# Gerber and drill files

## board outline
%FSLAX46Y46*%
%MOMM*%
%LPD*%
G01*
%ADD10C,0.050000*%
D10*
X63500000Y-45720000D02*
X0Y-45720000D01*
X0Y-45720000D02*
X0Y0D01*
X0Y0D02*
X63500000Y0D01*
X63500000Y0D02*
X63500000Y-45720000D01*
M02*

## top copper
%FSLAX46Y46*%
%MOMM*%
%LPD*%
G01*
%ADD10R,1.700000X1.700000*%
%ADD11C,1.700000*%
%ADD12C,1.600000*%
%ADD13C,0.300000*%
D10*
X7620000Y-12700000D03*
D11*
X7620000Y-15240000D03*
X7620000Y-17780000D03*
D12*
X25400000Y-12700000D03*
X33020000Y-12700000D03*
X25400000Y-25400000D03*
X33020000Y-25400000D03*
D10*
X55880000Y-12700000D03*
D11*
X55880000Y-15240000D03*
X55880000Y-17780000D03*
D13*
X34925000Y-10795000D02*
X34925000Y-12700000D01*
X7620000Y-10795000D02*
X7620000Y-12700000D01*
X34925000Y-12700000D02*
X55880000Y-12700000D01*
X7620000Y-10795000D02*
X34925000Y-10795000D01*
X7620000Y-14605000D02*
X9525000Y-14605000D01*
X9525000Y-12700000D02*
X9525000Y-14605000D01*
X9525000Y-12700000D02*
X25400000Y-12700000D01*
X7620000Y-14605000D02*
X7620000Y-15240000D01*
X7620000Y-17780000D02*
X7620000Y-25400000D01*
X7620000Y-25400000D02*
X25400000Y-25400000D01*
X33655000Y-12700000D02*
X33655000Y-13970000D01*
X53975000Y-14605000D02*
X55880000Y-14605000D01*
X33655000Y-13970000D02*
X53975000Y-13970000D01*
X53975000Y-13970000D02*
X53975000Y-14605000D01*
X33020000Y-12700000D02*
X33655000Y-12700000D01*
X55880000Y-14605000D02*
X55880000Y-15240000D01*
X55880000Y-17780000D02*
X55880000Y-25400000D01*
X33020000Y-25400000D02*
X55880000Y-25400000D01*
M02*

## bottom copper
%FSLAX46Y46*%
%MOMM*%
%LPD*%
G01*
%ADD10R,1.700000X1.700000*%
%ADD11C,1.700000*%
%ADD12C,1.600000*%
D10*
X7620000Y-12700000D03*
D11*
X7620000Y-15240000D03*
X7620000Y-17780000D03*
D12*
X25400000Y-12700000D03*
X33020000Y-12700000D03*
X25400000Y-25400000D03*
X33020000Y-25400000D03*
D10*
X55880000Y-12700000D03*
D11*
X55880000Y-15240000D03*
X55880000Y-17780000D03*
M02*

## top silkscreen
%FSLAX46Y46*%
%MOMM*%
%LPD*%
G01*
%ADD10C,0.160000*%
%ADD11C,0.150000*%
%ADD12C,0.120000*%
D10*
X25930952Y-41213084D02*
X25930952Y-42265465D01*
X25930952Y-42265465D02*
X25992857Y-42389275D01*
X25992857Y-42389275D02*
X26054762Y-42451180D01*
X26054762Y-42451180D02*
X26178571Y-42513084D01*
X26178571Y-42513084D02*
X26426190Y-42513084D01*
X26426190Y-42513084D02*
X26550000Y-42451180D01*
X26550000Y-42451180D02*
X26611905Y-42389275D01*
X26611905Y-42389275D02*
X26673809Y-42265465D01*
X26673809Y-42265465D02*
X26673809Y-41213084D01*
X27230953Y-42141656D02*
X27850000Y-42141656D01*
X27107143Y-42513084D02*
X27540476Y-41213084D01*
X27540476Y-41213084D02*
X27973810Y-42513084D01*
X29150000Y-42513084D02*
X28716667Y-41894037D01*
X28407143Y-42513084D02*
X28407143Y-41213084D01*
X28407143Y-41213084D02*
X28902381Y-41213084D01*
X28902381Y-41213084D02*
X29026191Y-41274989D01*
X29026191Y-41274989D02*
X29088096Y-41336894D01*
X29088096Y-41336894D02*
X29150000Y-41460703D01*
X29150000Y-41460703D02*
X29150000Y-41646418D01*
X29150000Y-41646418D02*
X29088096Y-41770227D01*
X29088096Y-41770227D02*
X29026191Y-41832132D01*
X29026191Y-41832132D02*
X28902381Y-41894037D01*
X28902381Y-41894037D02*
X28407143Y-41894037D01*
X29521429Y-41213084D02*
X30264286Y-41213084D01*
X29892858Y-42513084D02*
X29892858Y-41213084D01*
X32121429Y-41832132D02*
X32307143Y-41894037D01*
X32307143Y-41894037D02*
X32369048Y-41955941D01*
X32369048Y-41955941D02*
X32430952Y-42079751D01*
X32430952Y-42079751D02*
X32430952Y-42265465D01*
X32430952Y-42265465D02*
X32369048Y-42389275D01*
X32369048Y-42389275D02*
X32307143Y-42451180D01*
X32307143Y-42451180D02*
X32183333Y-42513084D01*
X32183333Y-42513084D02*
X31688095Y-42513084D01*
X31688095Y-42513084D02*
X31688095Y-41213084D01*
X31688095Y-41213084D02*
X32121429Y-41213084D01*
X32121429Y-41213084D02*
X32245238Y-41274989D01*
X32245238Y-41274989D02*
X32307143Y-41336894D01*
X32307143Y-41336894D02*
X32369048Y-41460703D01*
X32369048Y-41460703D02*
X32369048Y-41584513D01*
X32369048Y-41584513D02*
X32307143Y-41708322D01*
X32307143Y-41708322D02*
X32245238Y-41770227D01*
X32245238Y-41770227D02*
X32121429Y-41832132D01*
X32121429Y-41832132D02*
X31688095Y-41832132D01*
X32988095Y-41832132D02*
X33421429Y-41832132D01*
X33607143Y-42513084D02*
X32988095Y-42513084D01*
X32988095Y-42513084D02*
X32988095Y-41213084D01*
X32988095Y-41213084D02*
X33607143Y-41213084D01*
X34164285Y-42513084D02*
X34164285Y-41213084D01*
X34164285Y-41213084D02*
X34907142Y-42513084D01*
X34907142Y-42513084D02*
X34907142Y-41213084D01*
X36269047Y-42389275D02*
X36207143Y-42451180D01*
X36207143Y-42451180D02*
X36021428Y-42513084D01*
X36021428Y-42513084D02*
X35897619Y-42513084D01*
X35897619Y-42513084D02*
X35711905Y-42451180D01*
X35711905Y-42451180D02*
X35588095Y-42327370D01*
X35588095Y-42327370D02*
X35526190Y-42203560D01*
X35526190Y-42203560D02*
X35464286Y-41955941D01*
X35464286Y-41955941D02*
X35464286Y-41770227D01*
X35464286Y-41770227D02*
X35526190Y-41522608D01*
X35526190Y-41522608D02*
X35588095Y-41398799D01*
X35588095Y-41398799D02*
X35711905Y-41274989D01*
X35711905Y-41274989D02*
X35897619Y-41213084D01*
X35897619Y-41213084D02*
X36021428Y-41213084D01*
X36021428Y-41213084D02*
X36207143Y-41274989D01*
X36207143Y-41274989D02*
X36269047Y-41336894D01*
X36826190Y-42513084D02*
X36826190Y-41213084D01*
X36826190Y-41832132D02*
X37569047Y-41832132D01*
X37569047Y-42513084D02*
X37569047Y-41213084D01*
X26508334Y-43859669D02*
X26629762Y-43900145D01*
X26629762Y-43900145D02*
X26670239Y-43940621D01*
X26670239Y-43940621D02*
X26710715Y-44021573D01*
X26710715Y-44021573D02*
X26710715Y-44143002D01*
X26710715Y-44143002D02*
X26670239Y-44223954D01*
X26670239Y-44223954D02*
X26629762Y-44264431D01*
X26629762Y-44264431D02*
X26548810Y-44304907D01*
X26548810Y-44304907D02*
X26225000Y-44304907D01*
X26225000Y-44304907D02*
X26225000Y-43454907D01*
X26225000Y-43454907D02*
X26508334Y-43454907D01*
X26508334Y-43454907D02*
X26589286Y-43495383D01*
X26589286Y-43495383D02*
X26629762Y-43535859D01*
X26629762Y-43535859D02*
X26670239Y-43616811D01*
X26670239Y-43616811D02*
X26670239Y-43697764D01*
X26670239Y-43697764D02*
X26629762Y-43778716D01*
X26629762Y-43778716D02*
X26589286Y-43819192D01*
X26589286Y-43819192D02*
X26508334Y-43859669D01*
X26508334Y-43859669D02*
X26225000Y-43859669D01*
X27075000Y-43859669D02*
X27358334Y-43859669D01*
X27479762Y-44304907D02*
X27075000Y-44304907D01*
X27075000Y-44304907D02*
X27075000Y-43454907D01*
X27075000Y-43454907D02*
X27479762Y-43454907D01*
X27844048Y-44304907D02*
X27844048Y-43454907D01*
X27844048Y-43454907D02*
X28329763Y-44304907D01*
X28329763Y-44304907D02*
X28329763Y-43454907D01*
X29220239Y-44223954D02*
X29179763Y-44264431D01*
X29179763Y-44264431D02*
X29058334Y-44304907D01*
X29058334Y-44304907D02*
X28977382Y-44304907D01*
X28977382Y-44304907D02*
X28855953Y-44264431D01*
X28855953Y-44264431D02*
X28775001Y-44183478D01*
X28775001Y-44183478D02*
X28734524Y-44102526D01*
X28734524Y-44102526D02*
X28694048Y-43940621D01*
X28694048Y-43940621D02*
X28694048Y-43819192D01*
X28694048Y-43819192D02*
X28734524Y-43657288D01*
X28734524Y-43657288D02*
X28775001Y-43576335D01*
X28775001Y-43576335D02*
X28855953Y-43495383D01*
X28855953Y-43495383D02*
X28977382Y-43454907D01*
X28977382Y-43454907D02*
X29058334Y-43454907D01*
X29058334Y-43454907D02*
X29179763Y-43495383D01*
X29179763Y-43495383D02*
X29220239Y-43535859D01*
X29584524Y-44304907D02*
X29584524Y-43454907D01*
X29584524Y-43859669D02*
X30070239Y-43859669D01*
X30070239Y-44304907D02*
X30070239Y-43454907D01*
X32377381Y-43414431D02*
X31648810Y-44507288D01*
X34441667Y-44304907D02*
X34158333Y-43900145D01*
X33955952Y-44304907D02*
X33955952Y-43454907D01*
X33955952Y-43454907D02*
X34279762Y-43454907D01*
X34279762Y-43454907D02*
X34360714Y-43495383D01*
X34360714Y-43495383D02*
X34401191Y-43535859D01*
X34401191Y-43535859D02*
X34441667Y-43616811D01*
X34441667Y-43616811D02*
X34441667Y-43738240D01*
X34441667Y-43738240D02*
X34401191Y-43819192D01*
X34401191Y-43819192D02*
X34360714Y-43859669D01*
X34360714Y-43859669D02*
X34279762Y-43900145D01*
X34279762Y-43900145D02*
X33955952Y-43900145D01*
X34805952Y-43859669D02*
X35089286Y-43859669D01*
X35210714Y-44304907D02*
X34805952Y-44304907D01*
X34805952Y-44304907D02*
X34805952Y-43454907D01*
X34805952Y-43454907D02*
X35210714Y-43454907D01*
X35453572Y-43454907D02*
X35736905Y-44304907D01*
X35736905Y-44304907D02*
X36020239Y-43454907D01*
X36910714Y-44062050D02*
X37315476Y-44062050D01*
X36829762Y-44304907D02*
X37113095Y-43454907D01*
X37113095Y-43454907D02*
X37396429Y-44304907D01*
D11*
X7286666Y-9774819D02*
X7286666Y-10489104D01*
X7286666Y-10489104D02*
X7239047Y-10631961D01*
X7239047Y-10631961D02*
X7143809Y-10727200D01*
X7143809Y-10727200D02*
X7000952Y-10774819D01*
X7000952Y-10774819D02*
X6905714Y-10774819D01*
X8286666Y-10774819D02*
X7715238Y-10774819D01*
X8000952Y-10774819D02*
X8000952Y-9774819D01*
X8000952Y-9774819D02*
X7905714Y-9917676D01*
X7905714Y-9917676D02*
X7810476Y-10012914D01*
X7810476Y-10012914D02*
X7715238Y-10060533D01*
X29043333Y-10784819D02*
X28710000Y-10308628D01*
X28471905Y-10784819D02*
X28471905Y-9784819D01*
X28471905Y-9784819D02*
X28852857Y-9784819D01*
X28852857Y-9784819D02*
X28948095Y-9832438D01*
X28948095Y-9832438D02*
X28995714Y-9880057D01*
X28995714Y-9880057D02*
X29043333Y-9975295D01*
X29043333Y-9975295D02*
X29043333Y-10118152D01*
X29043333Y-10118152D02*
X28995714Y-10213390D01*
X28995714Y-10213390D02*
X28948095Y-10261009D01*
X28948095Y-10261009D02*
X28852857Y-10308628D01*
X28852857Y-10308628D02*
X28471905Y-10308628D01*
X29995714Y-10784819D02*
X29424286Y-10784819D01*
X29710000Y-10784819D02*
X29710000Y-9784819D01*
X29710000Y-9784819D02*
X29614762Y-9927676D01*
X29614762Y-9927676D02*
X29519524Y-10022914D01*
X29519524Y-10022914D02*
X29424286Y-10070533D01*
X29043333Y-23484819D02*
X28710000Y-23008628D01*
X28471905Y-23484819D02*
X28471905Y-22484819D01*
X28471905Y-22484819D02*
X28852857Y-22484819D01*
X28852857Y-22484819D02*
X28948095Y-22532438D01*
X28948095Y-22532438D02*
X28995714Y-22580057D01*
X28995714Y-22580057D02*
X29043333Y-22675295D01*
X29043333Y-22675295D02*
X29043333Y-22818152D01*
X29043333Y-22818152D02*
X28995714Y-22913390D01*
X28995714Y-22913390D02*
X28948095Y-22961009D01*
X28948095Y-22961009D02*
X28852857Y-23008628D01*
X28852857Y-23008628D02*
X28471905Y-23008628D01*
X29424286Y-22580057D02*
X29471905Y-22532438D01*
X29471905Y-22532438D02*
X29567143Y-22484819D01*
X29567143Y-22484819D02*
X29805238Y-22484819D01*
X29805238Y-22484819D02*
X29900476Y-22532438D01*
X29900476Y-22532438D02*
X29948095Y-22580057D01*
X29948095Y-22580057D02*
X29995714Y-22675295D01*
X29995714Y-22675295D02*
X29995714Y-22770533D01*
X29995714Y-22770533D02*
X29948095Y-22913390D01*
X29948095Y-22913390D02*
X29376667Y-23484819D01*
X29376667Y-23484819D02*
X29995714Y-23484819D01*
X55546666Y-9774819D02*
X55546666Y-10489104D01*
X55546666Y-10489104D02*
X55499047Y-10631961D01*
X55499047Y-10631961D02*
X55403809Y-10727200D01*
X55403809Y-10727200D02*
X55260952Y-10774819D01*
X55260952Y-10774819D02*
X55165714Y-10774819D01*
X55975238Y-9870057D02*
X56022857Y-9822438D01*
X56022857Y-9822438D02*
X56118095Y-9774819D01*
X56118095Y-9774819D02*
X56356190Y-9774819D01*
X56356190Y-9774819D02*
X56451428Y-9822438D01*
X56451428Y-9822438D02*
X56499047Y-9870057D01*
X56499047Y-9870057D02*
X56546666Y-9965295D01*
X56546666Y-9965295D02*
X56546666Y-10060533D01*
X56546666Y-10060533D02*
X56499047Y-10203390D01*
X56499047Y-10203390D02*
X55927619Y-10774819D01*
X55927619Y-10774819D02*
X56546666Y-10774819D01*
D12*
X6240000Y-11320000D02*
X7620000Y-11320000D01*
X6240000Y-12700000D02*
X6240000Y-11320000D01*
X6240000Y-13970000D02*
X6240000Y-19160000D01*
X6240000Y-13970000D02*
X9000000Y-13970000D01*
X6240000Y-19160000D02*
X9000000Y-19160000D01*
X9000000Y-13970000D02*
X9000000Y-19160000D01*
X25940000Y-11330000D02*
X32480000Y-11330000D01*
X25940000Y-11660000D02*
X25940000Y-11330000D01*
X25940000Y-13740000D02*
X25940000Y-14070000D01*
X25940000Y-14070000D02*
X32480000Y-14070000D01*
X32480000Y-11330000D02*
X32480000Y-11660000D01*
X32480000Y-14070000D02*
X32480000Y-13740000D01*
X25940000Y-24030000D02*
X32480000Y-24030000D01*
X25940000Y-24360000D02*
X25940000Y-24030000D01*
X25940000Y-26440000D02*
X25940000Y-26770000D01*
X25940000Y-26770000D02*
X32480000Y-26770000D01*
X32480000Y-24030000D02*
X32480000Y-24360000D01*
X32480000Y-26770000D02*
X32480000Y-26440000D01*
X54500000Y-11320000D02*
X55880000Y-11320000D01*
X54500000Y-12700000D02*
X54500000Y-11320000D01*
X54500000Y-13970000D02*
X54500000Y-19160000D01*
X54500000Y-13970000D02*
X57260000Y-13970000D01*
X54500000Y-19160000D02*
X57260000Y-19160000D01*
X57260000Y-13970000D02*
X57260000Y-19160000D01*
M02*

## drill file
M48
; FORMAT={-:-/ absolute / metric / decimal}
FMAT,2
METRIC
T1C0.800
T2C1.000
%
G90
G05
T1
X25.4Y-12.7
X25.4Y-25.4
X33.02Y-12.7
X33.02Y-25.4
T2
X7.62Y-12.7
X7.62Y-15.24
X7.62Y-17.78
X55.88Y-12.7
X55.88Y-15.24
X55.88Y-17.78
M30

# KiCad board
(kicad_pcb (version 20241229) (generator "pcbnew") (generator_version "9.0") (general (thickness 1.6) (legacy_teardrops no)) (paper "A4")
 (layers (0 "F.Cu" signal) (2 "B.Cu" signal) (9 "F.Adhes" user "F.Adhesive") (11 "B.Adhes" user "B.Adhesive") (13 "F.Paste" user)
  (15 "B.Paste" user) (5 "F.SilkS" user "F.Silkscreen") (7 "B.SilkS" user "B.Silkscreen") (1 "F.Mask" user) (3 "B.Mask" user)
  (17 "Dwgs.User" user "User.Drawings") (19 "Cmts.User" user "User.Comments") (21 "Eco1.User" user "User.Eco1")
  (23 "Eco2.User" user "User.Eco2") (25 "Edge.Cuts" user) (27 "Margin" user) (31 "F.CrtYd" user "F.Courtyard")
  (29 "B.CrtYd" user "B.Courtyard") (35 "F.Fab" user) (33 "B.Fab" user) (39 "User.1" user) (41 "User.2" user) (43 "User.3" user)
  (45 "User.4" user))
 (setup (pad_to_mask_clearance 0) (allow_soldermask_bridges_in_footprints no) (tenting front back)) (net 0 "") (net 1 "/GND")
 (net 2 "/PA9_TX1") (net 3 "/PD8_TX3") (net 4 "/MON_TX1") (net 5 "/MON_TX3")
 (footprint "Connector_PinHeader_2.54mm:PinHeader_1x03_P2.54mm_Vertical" (layer "F.Cu") (at 7.62 12.7)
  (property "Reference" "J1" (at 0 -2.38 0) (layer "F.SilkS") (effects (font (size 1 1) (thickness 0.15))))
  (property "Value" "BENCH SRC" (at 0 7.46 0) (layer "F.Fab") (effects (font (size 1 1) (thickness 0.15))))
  (fp_line (start -1.38 -1.38) (end 0 -1.38) (stroke (width 0.12) (type solid)) (layer "F.SilkS"))
  (fp_line (start -1.38 0) (end -1.38 -1.38) (stroke (width 0.12) (type solid)) (layer "F.SilkS"))
  (fp_line (start -1.38 1.27) (end -1.38 6.46) (stroke (width 0.12) (type solid)) (layer "F.SilkS"))
  (fp_line (start -1.38 1.27) (end 1.38 1.27) (stroke (width 0.12) (type solid)) (layer "F.SilkS"))
  (fp_line (start -1.38 6.46) (end 1.38 6.46) (stroke (width 0.12) (type solid)) (layer "F.SilkS"))
  (fp_line (start 1.38 1.27) (end 1.38 6.46) (stroke (width 0.12) (type solid)) (layer "F.SilkS"))
  (pad "1" thru_hole rect (at 0 0) (size 1.7 1.7) (drill 1) (layers "*.Cu" "*.Mask") (remove_unused_layers no) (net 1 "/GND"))
  (pad "2" thru_hole circle (at 0 2.54) (size 1.7 1.7) (drill 1) (layers "*.Cu" "*.Mask") (remove_unused_layers no) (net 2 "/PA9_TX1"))
  (pad "3" thru_hole circle (at 0 5.08) (size 1.7 1.7) (drill 1) (layers "*.Cu" "*.Mask") (remove_unused_layers no) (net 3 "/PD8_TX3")))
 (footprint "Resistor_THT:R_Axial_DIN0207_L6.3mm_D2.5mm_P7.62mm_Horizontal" (layer "F.Cu") (at 25.4 12.7)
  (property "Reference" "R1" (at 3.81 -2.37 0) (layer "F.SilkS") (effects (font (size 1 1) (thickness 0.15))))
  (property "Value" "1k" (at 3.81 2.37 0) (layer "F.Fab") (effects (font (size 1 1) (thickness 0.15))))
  (fp_line (start 0.54 -1.37) (end 7.08 -1.37) (stroke (width 0.12) (type solid)) (layer "F.SilkS"))
  (fp_line (start 0.54 -1.04) (end 0.54 -1.37) (stroke (width 0.12) (type solid)) (layer "F.SilkS"))
  (fp_line (start 0.54 1.04) (end 0.54 1.37) (stroke (width 0.12) (type solid)) (layer "F.SilkS"))
  (fp_line (start 0.54 1.37) (end 7.08 1.37) (stroke (width 0.12) (type solid)) (layer "F.SilkS"))
  (fp_line (start 7.08 -1.37) (end 7.08 -1.04) (stroke (width 0.12) (type solid)) (layer "F.SilkS"))
  (fp_line (start 7.08 1.37) (end 7.08 1.04) (stroke (width 0.12) (type solid)) (layer "F.SilkS"))
  (pad "1" thru_hole circle (at 0 0) (size 1.6 1.6) (drill 0.8) (layers "*.Cu" "*.Mask") (remove_unused_layers no) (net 2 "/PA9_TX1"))
  (pad "2" thru_hole circle (at 7.62 0) (size 1.6 1.6) (drill 0.8) (layers "*.Cu" "*.Mask") (remove_unused_layers no) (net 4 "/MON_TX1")))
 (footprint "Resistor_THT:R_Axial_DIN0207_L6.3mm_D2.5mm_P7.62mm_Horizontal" (layer "F.Cu") (at 25.4 25.4)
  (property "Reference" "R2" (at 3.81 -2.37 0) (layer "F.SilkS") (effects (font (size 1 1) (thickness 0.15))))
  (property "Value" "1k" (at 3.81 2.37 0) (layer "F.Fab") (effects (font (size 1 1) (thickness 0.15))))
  (fp_line (start 0.54 -1.37) (end 7.08 -1.37) (stroke (width 0.12) (type solid)) (layer "F.SilkS"))
  (fp_line (start 0.54 -1.04) (end 0.54 -1.37) (stroke (width 0.12) (type solid)) (layer "F.SilkS"))
  (fp_line (start 0.54 1.04) (end 0.54 1.37) (stroke (width 0.12) (type solid)) (layer "F.SilkS"))
  (fp_line (start 0.54 1.37) (end 7.08 1.37) (stroke (width 0.12) (type solid)) (layer "F.SilkS"))
  (fp_line (start 7.08 -1.37) (end 7.08 -1.04) (stroke (width 0.12) (type solid)) (layer "F.SilkS"))
  (fp_line (start 7.08 1.37) (end 7.08 1.04) (stroke (width 0.12) (type solid)) (layer "F.SilkS"))
  (pad "1" thru_hole circle (at 0 0) (size 1.6 1.6) (drill 0.8) (layers "*.Cu" "*.Mask") (remove_unused_layers no) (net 3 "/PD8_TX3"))
  (pad "2" thru_hole circle (at 7.62 0) (size 1.6 1.6) (drill 0.8) (layers "*.Cu" "*.Mask") (remove_unused_layers no) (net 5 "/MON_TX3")))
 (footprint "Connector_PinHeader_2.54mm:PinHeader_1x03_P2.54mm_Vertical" (layer "F.Cu") (at 55.88 12.7)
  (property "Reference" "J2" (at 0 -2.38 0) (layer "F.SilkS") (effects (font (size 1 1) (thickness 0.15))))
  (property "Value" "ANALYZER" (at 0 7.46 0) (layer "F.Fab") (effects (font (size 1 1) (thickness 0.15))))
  (fp_line (start -1.38 -1.38) (end 0 -1.38) (stroke (width 0.12) (type solid)) (layer "F.SilkS"))
  (fp_line (start -1.38 0) (end -1.38 -1.38) (stroke (width 0.12) (type solid)) (layer "F.SilkS"))
  (fp_line (start -1.38 1.27) (end -1.38 6.46) (stroke (width 0.12) (type solid)) (layer "F.SilkS"))
  (fp_line (start -1.38 1.27) (end 1.38 1.27) (stroke (width 0.12) (type solid)) (layer "F.SilkS"))
  (fp_line (start -1.38 6.46) (end 1.38 6.46) (stroke (width 0.12) (type solid)) (layer "F.SilkS"))
  (fp_line (start 1.38 1.27) (end 1.38 6.46) (stroke (width 0.12) (type solid)) (layer "F.SilkS"))
  (pad "1" thru_hole rect (at 0 0) (size 1.7 1.7) (drill 1) (layers "*.Cu" "*.Mask") (remove_unused_layers no) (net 1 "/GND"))
  (pad "2" thru_hole circle (at 0 2.54) (size 1.7 1.7) (drill 1) (layers "*.Cu" "*.Mask") (remove_unused_layers no) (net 4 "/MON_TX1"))
  (pad "3" thru_hole circle (at 0 5.08) (size 1.7 1.7) (drill 1) (layers "*.Cu" "*.Mask") (remove_unused_layers no) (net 5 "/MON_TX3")))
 (gr_line (start 63.5 45.72) (end 0 45.72) (stroke (width 0.05) (type default)) (layer "Edge.Cuts"))
 (gr_line (start 0 45.72) (end 0 0) (stroke (width 0.05) (type default)) (layer "Edge.Cuts"))
 (gr_line (start 0 0) (end 63.5 0) (stroke (width 0.05) (type default)) (layer "Edge.Cuts"))
 (gr_line (start 63.5 0) (end 63.5 45.72) (stroke (width 0.05) (type default)) (layer "Edge.Cuts"))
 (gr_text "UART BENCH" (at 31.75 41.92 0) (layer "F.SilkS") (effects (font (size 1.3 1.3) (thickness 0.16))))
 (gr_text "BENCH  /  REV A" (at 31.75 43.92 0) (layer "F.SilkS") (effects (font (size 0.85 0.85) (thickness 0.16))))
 (segment (start 34.925 10.795) (end 34.925 12.7) (width 0.3) (layer "F.Cu") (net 1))
 (segment (start 7.62 10.795) (end 7.62 12.7) (width 0.3) (layer "F.Cu") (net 1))
 (segment (start 34.925 12.7) (end 55.88 12.7) (width 0.3) (layer "F.Cu") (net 1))
 (segment (start 7.62 10.795) (end 34.925 10.795) (width 0.3) (layer "F.Cu") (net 1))
 (segment (start 7.62 14.605) (end 9.525 14.605) (width 0.3) (layer "F.Cu") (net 2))
 (segment (start 9.525 12.7) (end 9.525 14.605) (width 0.3) (layer "F.Cu") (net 2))
 (segment (start 9.525 12.7) (end 25.4 12.7) (width 0.3) (layer "F.Cu") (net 2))
 (segment (start 7.62 14.605) (end 7.62 15.24) (width 0.3) (layer "F.Cu") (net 2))
 (segment (start 7.62 17.78) (end 7.62 25.4) (width 0.3) (layer "F.Cu") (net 3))
 (segment (start 7.62 25.4) (end 25.4 25.4) (width 0.3) (layer "F.Cu") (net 3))
 (segment (start 33.655 12.7) (end 33.655 13.97) (width 0.3) (layer "F.Cu") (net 4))
 (segment (start 53.975 14.605) (end 55.88 14.605) (width 0.3) (layer "F.Cu") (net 4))
 (segment (start 33.655 13.97) (end 53.975 13.97) (width 0.3) (layer "F.Cu") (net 4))
 (segment (start 53.975 13.97) (end 53.975 14.605) (width 0.3) (layer "F.Cu") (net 4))
 (segment (start 33.02 12.7) (end 33.655 12.7) (width 0.3) (layer "F.Cu") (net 4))
 (segment (start 55.88 14.605) (end 55.88 15.24) (width 0.3) (layer "F.Cu") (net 4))
 (segment (start 55.88 17.78) (end 55.88 25.4) (width 0.3) (layer "F.Cu") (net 5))
 (segment (start 33.02 25.4) (end 55.88 25.4) (width 0.3) (layer "F.Cu") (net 5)))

